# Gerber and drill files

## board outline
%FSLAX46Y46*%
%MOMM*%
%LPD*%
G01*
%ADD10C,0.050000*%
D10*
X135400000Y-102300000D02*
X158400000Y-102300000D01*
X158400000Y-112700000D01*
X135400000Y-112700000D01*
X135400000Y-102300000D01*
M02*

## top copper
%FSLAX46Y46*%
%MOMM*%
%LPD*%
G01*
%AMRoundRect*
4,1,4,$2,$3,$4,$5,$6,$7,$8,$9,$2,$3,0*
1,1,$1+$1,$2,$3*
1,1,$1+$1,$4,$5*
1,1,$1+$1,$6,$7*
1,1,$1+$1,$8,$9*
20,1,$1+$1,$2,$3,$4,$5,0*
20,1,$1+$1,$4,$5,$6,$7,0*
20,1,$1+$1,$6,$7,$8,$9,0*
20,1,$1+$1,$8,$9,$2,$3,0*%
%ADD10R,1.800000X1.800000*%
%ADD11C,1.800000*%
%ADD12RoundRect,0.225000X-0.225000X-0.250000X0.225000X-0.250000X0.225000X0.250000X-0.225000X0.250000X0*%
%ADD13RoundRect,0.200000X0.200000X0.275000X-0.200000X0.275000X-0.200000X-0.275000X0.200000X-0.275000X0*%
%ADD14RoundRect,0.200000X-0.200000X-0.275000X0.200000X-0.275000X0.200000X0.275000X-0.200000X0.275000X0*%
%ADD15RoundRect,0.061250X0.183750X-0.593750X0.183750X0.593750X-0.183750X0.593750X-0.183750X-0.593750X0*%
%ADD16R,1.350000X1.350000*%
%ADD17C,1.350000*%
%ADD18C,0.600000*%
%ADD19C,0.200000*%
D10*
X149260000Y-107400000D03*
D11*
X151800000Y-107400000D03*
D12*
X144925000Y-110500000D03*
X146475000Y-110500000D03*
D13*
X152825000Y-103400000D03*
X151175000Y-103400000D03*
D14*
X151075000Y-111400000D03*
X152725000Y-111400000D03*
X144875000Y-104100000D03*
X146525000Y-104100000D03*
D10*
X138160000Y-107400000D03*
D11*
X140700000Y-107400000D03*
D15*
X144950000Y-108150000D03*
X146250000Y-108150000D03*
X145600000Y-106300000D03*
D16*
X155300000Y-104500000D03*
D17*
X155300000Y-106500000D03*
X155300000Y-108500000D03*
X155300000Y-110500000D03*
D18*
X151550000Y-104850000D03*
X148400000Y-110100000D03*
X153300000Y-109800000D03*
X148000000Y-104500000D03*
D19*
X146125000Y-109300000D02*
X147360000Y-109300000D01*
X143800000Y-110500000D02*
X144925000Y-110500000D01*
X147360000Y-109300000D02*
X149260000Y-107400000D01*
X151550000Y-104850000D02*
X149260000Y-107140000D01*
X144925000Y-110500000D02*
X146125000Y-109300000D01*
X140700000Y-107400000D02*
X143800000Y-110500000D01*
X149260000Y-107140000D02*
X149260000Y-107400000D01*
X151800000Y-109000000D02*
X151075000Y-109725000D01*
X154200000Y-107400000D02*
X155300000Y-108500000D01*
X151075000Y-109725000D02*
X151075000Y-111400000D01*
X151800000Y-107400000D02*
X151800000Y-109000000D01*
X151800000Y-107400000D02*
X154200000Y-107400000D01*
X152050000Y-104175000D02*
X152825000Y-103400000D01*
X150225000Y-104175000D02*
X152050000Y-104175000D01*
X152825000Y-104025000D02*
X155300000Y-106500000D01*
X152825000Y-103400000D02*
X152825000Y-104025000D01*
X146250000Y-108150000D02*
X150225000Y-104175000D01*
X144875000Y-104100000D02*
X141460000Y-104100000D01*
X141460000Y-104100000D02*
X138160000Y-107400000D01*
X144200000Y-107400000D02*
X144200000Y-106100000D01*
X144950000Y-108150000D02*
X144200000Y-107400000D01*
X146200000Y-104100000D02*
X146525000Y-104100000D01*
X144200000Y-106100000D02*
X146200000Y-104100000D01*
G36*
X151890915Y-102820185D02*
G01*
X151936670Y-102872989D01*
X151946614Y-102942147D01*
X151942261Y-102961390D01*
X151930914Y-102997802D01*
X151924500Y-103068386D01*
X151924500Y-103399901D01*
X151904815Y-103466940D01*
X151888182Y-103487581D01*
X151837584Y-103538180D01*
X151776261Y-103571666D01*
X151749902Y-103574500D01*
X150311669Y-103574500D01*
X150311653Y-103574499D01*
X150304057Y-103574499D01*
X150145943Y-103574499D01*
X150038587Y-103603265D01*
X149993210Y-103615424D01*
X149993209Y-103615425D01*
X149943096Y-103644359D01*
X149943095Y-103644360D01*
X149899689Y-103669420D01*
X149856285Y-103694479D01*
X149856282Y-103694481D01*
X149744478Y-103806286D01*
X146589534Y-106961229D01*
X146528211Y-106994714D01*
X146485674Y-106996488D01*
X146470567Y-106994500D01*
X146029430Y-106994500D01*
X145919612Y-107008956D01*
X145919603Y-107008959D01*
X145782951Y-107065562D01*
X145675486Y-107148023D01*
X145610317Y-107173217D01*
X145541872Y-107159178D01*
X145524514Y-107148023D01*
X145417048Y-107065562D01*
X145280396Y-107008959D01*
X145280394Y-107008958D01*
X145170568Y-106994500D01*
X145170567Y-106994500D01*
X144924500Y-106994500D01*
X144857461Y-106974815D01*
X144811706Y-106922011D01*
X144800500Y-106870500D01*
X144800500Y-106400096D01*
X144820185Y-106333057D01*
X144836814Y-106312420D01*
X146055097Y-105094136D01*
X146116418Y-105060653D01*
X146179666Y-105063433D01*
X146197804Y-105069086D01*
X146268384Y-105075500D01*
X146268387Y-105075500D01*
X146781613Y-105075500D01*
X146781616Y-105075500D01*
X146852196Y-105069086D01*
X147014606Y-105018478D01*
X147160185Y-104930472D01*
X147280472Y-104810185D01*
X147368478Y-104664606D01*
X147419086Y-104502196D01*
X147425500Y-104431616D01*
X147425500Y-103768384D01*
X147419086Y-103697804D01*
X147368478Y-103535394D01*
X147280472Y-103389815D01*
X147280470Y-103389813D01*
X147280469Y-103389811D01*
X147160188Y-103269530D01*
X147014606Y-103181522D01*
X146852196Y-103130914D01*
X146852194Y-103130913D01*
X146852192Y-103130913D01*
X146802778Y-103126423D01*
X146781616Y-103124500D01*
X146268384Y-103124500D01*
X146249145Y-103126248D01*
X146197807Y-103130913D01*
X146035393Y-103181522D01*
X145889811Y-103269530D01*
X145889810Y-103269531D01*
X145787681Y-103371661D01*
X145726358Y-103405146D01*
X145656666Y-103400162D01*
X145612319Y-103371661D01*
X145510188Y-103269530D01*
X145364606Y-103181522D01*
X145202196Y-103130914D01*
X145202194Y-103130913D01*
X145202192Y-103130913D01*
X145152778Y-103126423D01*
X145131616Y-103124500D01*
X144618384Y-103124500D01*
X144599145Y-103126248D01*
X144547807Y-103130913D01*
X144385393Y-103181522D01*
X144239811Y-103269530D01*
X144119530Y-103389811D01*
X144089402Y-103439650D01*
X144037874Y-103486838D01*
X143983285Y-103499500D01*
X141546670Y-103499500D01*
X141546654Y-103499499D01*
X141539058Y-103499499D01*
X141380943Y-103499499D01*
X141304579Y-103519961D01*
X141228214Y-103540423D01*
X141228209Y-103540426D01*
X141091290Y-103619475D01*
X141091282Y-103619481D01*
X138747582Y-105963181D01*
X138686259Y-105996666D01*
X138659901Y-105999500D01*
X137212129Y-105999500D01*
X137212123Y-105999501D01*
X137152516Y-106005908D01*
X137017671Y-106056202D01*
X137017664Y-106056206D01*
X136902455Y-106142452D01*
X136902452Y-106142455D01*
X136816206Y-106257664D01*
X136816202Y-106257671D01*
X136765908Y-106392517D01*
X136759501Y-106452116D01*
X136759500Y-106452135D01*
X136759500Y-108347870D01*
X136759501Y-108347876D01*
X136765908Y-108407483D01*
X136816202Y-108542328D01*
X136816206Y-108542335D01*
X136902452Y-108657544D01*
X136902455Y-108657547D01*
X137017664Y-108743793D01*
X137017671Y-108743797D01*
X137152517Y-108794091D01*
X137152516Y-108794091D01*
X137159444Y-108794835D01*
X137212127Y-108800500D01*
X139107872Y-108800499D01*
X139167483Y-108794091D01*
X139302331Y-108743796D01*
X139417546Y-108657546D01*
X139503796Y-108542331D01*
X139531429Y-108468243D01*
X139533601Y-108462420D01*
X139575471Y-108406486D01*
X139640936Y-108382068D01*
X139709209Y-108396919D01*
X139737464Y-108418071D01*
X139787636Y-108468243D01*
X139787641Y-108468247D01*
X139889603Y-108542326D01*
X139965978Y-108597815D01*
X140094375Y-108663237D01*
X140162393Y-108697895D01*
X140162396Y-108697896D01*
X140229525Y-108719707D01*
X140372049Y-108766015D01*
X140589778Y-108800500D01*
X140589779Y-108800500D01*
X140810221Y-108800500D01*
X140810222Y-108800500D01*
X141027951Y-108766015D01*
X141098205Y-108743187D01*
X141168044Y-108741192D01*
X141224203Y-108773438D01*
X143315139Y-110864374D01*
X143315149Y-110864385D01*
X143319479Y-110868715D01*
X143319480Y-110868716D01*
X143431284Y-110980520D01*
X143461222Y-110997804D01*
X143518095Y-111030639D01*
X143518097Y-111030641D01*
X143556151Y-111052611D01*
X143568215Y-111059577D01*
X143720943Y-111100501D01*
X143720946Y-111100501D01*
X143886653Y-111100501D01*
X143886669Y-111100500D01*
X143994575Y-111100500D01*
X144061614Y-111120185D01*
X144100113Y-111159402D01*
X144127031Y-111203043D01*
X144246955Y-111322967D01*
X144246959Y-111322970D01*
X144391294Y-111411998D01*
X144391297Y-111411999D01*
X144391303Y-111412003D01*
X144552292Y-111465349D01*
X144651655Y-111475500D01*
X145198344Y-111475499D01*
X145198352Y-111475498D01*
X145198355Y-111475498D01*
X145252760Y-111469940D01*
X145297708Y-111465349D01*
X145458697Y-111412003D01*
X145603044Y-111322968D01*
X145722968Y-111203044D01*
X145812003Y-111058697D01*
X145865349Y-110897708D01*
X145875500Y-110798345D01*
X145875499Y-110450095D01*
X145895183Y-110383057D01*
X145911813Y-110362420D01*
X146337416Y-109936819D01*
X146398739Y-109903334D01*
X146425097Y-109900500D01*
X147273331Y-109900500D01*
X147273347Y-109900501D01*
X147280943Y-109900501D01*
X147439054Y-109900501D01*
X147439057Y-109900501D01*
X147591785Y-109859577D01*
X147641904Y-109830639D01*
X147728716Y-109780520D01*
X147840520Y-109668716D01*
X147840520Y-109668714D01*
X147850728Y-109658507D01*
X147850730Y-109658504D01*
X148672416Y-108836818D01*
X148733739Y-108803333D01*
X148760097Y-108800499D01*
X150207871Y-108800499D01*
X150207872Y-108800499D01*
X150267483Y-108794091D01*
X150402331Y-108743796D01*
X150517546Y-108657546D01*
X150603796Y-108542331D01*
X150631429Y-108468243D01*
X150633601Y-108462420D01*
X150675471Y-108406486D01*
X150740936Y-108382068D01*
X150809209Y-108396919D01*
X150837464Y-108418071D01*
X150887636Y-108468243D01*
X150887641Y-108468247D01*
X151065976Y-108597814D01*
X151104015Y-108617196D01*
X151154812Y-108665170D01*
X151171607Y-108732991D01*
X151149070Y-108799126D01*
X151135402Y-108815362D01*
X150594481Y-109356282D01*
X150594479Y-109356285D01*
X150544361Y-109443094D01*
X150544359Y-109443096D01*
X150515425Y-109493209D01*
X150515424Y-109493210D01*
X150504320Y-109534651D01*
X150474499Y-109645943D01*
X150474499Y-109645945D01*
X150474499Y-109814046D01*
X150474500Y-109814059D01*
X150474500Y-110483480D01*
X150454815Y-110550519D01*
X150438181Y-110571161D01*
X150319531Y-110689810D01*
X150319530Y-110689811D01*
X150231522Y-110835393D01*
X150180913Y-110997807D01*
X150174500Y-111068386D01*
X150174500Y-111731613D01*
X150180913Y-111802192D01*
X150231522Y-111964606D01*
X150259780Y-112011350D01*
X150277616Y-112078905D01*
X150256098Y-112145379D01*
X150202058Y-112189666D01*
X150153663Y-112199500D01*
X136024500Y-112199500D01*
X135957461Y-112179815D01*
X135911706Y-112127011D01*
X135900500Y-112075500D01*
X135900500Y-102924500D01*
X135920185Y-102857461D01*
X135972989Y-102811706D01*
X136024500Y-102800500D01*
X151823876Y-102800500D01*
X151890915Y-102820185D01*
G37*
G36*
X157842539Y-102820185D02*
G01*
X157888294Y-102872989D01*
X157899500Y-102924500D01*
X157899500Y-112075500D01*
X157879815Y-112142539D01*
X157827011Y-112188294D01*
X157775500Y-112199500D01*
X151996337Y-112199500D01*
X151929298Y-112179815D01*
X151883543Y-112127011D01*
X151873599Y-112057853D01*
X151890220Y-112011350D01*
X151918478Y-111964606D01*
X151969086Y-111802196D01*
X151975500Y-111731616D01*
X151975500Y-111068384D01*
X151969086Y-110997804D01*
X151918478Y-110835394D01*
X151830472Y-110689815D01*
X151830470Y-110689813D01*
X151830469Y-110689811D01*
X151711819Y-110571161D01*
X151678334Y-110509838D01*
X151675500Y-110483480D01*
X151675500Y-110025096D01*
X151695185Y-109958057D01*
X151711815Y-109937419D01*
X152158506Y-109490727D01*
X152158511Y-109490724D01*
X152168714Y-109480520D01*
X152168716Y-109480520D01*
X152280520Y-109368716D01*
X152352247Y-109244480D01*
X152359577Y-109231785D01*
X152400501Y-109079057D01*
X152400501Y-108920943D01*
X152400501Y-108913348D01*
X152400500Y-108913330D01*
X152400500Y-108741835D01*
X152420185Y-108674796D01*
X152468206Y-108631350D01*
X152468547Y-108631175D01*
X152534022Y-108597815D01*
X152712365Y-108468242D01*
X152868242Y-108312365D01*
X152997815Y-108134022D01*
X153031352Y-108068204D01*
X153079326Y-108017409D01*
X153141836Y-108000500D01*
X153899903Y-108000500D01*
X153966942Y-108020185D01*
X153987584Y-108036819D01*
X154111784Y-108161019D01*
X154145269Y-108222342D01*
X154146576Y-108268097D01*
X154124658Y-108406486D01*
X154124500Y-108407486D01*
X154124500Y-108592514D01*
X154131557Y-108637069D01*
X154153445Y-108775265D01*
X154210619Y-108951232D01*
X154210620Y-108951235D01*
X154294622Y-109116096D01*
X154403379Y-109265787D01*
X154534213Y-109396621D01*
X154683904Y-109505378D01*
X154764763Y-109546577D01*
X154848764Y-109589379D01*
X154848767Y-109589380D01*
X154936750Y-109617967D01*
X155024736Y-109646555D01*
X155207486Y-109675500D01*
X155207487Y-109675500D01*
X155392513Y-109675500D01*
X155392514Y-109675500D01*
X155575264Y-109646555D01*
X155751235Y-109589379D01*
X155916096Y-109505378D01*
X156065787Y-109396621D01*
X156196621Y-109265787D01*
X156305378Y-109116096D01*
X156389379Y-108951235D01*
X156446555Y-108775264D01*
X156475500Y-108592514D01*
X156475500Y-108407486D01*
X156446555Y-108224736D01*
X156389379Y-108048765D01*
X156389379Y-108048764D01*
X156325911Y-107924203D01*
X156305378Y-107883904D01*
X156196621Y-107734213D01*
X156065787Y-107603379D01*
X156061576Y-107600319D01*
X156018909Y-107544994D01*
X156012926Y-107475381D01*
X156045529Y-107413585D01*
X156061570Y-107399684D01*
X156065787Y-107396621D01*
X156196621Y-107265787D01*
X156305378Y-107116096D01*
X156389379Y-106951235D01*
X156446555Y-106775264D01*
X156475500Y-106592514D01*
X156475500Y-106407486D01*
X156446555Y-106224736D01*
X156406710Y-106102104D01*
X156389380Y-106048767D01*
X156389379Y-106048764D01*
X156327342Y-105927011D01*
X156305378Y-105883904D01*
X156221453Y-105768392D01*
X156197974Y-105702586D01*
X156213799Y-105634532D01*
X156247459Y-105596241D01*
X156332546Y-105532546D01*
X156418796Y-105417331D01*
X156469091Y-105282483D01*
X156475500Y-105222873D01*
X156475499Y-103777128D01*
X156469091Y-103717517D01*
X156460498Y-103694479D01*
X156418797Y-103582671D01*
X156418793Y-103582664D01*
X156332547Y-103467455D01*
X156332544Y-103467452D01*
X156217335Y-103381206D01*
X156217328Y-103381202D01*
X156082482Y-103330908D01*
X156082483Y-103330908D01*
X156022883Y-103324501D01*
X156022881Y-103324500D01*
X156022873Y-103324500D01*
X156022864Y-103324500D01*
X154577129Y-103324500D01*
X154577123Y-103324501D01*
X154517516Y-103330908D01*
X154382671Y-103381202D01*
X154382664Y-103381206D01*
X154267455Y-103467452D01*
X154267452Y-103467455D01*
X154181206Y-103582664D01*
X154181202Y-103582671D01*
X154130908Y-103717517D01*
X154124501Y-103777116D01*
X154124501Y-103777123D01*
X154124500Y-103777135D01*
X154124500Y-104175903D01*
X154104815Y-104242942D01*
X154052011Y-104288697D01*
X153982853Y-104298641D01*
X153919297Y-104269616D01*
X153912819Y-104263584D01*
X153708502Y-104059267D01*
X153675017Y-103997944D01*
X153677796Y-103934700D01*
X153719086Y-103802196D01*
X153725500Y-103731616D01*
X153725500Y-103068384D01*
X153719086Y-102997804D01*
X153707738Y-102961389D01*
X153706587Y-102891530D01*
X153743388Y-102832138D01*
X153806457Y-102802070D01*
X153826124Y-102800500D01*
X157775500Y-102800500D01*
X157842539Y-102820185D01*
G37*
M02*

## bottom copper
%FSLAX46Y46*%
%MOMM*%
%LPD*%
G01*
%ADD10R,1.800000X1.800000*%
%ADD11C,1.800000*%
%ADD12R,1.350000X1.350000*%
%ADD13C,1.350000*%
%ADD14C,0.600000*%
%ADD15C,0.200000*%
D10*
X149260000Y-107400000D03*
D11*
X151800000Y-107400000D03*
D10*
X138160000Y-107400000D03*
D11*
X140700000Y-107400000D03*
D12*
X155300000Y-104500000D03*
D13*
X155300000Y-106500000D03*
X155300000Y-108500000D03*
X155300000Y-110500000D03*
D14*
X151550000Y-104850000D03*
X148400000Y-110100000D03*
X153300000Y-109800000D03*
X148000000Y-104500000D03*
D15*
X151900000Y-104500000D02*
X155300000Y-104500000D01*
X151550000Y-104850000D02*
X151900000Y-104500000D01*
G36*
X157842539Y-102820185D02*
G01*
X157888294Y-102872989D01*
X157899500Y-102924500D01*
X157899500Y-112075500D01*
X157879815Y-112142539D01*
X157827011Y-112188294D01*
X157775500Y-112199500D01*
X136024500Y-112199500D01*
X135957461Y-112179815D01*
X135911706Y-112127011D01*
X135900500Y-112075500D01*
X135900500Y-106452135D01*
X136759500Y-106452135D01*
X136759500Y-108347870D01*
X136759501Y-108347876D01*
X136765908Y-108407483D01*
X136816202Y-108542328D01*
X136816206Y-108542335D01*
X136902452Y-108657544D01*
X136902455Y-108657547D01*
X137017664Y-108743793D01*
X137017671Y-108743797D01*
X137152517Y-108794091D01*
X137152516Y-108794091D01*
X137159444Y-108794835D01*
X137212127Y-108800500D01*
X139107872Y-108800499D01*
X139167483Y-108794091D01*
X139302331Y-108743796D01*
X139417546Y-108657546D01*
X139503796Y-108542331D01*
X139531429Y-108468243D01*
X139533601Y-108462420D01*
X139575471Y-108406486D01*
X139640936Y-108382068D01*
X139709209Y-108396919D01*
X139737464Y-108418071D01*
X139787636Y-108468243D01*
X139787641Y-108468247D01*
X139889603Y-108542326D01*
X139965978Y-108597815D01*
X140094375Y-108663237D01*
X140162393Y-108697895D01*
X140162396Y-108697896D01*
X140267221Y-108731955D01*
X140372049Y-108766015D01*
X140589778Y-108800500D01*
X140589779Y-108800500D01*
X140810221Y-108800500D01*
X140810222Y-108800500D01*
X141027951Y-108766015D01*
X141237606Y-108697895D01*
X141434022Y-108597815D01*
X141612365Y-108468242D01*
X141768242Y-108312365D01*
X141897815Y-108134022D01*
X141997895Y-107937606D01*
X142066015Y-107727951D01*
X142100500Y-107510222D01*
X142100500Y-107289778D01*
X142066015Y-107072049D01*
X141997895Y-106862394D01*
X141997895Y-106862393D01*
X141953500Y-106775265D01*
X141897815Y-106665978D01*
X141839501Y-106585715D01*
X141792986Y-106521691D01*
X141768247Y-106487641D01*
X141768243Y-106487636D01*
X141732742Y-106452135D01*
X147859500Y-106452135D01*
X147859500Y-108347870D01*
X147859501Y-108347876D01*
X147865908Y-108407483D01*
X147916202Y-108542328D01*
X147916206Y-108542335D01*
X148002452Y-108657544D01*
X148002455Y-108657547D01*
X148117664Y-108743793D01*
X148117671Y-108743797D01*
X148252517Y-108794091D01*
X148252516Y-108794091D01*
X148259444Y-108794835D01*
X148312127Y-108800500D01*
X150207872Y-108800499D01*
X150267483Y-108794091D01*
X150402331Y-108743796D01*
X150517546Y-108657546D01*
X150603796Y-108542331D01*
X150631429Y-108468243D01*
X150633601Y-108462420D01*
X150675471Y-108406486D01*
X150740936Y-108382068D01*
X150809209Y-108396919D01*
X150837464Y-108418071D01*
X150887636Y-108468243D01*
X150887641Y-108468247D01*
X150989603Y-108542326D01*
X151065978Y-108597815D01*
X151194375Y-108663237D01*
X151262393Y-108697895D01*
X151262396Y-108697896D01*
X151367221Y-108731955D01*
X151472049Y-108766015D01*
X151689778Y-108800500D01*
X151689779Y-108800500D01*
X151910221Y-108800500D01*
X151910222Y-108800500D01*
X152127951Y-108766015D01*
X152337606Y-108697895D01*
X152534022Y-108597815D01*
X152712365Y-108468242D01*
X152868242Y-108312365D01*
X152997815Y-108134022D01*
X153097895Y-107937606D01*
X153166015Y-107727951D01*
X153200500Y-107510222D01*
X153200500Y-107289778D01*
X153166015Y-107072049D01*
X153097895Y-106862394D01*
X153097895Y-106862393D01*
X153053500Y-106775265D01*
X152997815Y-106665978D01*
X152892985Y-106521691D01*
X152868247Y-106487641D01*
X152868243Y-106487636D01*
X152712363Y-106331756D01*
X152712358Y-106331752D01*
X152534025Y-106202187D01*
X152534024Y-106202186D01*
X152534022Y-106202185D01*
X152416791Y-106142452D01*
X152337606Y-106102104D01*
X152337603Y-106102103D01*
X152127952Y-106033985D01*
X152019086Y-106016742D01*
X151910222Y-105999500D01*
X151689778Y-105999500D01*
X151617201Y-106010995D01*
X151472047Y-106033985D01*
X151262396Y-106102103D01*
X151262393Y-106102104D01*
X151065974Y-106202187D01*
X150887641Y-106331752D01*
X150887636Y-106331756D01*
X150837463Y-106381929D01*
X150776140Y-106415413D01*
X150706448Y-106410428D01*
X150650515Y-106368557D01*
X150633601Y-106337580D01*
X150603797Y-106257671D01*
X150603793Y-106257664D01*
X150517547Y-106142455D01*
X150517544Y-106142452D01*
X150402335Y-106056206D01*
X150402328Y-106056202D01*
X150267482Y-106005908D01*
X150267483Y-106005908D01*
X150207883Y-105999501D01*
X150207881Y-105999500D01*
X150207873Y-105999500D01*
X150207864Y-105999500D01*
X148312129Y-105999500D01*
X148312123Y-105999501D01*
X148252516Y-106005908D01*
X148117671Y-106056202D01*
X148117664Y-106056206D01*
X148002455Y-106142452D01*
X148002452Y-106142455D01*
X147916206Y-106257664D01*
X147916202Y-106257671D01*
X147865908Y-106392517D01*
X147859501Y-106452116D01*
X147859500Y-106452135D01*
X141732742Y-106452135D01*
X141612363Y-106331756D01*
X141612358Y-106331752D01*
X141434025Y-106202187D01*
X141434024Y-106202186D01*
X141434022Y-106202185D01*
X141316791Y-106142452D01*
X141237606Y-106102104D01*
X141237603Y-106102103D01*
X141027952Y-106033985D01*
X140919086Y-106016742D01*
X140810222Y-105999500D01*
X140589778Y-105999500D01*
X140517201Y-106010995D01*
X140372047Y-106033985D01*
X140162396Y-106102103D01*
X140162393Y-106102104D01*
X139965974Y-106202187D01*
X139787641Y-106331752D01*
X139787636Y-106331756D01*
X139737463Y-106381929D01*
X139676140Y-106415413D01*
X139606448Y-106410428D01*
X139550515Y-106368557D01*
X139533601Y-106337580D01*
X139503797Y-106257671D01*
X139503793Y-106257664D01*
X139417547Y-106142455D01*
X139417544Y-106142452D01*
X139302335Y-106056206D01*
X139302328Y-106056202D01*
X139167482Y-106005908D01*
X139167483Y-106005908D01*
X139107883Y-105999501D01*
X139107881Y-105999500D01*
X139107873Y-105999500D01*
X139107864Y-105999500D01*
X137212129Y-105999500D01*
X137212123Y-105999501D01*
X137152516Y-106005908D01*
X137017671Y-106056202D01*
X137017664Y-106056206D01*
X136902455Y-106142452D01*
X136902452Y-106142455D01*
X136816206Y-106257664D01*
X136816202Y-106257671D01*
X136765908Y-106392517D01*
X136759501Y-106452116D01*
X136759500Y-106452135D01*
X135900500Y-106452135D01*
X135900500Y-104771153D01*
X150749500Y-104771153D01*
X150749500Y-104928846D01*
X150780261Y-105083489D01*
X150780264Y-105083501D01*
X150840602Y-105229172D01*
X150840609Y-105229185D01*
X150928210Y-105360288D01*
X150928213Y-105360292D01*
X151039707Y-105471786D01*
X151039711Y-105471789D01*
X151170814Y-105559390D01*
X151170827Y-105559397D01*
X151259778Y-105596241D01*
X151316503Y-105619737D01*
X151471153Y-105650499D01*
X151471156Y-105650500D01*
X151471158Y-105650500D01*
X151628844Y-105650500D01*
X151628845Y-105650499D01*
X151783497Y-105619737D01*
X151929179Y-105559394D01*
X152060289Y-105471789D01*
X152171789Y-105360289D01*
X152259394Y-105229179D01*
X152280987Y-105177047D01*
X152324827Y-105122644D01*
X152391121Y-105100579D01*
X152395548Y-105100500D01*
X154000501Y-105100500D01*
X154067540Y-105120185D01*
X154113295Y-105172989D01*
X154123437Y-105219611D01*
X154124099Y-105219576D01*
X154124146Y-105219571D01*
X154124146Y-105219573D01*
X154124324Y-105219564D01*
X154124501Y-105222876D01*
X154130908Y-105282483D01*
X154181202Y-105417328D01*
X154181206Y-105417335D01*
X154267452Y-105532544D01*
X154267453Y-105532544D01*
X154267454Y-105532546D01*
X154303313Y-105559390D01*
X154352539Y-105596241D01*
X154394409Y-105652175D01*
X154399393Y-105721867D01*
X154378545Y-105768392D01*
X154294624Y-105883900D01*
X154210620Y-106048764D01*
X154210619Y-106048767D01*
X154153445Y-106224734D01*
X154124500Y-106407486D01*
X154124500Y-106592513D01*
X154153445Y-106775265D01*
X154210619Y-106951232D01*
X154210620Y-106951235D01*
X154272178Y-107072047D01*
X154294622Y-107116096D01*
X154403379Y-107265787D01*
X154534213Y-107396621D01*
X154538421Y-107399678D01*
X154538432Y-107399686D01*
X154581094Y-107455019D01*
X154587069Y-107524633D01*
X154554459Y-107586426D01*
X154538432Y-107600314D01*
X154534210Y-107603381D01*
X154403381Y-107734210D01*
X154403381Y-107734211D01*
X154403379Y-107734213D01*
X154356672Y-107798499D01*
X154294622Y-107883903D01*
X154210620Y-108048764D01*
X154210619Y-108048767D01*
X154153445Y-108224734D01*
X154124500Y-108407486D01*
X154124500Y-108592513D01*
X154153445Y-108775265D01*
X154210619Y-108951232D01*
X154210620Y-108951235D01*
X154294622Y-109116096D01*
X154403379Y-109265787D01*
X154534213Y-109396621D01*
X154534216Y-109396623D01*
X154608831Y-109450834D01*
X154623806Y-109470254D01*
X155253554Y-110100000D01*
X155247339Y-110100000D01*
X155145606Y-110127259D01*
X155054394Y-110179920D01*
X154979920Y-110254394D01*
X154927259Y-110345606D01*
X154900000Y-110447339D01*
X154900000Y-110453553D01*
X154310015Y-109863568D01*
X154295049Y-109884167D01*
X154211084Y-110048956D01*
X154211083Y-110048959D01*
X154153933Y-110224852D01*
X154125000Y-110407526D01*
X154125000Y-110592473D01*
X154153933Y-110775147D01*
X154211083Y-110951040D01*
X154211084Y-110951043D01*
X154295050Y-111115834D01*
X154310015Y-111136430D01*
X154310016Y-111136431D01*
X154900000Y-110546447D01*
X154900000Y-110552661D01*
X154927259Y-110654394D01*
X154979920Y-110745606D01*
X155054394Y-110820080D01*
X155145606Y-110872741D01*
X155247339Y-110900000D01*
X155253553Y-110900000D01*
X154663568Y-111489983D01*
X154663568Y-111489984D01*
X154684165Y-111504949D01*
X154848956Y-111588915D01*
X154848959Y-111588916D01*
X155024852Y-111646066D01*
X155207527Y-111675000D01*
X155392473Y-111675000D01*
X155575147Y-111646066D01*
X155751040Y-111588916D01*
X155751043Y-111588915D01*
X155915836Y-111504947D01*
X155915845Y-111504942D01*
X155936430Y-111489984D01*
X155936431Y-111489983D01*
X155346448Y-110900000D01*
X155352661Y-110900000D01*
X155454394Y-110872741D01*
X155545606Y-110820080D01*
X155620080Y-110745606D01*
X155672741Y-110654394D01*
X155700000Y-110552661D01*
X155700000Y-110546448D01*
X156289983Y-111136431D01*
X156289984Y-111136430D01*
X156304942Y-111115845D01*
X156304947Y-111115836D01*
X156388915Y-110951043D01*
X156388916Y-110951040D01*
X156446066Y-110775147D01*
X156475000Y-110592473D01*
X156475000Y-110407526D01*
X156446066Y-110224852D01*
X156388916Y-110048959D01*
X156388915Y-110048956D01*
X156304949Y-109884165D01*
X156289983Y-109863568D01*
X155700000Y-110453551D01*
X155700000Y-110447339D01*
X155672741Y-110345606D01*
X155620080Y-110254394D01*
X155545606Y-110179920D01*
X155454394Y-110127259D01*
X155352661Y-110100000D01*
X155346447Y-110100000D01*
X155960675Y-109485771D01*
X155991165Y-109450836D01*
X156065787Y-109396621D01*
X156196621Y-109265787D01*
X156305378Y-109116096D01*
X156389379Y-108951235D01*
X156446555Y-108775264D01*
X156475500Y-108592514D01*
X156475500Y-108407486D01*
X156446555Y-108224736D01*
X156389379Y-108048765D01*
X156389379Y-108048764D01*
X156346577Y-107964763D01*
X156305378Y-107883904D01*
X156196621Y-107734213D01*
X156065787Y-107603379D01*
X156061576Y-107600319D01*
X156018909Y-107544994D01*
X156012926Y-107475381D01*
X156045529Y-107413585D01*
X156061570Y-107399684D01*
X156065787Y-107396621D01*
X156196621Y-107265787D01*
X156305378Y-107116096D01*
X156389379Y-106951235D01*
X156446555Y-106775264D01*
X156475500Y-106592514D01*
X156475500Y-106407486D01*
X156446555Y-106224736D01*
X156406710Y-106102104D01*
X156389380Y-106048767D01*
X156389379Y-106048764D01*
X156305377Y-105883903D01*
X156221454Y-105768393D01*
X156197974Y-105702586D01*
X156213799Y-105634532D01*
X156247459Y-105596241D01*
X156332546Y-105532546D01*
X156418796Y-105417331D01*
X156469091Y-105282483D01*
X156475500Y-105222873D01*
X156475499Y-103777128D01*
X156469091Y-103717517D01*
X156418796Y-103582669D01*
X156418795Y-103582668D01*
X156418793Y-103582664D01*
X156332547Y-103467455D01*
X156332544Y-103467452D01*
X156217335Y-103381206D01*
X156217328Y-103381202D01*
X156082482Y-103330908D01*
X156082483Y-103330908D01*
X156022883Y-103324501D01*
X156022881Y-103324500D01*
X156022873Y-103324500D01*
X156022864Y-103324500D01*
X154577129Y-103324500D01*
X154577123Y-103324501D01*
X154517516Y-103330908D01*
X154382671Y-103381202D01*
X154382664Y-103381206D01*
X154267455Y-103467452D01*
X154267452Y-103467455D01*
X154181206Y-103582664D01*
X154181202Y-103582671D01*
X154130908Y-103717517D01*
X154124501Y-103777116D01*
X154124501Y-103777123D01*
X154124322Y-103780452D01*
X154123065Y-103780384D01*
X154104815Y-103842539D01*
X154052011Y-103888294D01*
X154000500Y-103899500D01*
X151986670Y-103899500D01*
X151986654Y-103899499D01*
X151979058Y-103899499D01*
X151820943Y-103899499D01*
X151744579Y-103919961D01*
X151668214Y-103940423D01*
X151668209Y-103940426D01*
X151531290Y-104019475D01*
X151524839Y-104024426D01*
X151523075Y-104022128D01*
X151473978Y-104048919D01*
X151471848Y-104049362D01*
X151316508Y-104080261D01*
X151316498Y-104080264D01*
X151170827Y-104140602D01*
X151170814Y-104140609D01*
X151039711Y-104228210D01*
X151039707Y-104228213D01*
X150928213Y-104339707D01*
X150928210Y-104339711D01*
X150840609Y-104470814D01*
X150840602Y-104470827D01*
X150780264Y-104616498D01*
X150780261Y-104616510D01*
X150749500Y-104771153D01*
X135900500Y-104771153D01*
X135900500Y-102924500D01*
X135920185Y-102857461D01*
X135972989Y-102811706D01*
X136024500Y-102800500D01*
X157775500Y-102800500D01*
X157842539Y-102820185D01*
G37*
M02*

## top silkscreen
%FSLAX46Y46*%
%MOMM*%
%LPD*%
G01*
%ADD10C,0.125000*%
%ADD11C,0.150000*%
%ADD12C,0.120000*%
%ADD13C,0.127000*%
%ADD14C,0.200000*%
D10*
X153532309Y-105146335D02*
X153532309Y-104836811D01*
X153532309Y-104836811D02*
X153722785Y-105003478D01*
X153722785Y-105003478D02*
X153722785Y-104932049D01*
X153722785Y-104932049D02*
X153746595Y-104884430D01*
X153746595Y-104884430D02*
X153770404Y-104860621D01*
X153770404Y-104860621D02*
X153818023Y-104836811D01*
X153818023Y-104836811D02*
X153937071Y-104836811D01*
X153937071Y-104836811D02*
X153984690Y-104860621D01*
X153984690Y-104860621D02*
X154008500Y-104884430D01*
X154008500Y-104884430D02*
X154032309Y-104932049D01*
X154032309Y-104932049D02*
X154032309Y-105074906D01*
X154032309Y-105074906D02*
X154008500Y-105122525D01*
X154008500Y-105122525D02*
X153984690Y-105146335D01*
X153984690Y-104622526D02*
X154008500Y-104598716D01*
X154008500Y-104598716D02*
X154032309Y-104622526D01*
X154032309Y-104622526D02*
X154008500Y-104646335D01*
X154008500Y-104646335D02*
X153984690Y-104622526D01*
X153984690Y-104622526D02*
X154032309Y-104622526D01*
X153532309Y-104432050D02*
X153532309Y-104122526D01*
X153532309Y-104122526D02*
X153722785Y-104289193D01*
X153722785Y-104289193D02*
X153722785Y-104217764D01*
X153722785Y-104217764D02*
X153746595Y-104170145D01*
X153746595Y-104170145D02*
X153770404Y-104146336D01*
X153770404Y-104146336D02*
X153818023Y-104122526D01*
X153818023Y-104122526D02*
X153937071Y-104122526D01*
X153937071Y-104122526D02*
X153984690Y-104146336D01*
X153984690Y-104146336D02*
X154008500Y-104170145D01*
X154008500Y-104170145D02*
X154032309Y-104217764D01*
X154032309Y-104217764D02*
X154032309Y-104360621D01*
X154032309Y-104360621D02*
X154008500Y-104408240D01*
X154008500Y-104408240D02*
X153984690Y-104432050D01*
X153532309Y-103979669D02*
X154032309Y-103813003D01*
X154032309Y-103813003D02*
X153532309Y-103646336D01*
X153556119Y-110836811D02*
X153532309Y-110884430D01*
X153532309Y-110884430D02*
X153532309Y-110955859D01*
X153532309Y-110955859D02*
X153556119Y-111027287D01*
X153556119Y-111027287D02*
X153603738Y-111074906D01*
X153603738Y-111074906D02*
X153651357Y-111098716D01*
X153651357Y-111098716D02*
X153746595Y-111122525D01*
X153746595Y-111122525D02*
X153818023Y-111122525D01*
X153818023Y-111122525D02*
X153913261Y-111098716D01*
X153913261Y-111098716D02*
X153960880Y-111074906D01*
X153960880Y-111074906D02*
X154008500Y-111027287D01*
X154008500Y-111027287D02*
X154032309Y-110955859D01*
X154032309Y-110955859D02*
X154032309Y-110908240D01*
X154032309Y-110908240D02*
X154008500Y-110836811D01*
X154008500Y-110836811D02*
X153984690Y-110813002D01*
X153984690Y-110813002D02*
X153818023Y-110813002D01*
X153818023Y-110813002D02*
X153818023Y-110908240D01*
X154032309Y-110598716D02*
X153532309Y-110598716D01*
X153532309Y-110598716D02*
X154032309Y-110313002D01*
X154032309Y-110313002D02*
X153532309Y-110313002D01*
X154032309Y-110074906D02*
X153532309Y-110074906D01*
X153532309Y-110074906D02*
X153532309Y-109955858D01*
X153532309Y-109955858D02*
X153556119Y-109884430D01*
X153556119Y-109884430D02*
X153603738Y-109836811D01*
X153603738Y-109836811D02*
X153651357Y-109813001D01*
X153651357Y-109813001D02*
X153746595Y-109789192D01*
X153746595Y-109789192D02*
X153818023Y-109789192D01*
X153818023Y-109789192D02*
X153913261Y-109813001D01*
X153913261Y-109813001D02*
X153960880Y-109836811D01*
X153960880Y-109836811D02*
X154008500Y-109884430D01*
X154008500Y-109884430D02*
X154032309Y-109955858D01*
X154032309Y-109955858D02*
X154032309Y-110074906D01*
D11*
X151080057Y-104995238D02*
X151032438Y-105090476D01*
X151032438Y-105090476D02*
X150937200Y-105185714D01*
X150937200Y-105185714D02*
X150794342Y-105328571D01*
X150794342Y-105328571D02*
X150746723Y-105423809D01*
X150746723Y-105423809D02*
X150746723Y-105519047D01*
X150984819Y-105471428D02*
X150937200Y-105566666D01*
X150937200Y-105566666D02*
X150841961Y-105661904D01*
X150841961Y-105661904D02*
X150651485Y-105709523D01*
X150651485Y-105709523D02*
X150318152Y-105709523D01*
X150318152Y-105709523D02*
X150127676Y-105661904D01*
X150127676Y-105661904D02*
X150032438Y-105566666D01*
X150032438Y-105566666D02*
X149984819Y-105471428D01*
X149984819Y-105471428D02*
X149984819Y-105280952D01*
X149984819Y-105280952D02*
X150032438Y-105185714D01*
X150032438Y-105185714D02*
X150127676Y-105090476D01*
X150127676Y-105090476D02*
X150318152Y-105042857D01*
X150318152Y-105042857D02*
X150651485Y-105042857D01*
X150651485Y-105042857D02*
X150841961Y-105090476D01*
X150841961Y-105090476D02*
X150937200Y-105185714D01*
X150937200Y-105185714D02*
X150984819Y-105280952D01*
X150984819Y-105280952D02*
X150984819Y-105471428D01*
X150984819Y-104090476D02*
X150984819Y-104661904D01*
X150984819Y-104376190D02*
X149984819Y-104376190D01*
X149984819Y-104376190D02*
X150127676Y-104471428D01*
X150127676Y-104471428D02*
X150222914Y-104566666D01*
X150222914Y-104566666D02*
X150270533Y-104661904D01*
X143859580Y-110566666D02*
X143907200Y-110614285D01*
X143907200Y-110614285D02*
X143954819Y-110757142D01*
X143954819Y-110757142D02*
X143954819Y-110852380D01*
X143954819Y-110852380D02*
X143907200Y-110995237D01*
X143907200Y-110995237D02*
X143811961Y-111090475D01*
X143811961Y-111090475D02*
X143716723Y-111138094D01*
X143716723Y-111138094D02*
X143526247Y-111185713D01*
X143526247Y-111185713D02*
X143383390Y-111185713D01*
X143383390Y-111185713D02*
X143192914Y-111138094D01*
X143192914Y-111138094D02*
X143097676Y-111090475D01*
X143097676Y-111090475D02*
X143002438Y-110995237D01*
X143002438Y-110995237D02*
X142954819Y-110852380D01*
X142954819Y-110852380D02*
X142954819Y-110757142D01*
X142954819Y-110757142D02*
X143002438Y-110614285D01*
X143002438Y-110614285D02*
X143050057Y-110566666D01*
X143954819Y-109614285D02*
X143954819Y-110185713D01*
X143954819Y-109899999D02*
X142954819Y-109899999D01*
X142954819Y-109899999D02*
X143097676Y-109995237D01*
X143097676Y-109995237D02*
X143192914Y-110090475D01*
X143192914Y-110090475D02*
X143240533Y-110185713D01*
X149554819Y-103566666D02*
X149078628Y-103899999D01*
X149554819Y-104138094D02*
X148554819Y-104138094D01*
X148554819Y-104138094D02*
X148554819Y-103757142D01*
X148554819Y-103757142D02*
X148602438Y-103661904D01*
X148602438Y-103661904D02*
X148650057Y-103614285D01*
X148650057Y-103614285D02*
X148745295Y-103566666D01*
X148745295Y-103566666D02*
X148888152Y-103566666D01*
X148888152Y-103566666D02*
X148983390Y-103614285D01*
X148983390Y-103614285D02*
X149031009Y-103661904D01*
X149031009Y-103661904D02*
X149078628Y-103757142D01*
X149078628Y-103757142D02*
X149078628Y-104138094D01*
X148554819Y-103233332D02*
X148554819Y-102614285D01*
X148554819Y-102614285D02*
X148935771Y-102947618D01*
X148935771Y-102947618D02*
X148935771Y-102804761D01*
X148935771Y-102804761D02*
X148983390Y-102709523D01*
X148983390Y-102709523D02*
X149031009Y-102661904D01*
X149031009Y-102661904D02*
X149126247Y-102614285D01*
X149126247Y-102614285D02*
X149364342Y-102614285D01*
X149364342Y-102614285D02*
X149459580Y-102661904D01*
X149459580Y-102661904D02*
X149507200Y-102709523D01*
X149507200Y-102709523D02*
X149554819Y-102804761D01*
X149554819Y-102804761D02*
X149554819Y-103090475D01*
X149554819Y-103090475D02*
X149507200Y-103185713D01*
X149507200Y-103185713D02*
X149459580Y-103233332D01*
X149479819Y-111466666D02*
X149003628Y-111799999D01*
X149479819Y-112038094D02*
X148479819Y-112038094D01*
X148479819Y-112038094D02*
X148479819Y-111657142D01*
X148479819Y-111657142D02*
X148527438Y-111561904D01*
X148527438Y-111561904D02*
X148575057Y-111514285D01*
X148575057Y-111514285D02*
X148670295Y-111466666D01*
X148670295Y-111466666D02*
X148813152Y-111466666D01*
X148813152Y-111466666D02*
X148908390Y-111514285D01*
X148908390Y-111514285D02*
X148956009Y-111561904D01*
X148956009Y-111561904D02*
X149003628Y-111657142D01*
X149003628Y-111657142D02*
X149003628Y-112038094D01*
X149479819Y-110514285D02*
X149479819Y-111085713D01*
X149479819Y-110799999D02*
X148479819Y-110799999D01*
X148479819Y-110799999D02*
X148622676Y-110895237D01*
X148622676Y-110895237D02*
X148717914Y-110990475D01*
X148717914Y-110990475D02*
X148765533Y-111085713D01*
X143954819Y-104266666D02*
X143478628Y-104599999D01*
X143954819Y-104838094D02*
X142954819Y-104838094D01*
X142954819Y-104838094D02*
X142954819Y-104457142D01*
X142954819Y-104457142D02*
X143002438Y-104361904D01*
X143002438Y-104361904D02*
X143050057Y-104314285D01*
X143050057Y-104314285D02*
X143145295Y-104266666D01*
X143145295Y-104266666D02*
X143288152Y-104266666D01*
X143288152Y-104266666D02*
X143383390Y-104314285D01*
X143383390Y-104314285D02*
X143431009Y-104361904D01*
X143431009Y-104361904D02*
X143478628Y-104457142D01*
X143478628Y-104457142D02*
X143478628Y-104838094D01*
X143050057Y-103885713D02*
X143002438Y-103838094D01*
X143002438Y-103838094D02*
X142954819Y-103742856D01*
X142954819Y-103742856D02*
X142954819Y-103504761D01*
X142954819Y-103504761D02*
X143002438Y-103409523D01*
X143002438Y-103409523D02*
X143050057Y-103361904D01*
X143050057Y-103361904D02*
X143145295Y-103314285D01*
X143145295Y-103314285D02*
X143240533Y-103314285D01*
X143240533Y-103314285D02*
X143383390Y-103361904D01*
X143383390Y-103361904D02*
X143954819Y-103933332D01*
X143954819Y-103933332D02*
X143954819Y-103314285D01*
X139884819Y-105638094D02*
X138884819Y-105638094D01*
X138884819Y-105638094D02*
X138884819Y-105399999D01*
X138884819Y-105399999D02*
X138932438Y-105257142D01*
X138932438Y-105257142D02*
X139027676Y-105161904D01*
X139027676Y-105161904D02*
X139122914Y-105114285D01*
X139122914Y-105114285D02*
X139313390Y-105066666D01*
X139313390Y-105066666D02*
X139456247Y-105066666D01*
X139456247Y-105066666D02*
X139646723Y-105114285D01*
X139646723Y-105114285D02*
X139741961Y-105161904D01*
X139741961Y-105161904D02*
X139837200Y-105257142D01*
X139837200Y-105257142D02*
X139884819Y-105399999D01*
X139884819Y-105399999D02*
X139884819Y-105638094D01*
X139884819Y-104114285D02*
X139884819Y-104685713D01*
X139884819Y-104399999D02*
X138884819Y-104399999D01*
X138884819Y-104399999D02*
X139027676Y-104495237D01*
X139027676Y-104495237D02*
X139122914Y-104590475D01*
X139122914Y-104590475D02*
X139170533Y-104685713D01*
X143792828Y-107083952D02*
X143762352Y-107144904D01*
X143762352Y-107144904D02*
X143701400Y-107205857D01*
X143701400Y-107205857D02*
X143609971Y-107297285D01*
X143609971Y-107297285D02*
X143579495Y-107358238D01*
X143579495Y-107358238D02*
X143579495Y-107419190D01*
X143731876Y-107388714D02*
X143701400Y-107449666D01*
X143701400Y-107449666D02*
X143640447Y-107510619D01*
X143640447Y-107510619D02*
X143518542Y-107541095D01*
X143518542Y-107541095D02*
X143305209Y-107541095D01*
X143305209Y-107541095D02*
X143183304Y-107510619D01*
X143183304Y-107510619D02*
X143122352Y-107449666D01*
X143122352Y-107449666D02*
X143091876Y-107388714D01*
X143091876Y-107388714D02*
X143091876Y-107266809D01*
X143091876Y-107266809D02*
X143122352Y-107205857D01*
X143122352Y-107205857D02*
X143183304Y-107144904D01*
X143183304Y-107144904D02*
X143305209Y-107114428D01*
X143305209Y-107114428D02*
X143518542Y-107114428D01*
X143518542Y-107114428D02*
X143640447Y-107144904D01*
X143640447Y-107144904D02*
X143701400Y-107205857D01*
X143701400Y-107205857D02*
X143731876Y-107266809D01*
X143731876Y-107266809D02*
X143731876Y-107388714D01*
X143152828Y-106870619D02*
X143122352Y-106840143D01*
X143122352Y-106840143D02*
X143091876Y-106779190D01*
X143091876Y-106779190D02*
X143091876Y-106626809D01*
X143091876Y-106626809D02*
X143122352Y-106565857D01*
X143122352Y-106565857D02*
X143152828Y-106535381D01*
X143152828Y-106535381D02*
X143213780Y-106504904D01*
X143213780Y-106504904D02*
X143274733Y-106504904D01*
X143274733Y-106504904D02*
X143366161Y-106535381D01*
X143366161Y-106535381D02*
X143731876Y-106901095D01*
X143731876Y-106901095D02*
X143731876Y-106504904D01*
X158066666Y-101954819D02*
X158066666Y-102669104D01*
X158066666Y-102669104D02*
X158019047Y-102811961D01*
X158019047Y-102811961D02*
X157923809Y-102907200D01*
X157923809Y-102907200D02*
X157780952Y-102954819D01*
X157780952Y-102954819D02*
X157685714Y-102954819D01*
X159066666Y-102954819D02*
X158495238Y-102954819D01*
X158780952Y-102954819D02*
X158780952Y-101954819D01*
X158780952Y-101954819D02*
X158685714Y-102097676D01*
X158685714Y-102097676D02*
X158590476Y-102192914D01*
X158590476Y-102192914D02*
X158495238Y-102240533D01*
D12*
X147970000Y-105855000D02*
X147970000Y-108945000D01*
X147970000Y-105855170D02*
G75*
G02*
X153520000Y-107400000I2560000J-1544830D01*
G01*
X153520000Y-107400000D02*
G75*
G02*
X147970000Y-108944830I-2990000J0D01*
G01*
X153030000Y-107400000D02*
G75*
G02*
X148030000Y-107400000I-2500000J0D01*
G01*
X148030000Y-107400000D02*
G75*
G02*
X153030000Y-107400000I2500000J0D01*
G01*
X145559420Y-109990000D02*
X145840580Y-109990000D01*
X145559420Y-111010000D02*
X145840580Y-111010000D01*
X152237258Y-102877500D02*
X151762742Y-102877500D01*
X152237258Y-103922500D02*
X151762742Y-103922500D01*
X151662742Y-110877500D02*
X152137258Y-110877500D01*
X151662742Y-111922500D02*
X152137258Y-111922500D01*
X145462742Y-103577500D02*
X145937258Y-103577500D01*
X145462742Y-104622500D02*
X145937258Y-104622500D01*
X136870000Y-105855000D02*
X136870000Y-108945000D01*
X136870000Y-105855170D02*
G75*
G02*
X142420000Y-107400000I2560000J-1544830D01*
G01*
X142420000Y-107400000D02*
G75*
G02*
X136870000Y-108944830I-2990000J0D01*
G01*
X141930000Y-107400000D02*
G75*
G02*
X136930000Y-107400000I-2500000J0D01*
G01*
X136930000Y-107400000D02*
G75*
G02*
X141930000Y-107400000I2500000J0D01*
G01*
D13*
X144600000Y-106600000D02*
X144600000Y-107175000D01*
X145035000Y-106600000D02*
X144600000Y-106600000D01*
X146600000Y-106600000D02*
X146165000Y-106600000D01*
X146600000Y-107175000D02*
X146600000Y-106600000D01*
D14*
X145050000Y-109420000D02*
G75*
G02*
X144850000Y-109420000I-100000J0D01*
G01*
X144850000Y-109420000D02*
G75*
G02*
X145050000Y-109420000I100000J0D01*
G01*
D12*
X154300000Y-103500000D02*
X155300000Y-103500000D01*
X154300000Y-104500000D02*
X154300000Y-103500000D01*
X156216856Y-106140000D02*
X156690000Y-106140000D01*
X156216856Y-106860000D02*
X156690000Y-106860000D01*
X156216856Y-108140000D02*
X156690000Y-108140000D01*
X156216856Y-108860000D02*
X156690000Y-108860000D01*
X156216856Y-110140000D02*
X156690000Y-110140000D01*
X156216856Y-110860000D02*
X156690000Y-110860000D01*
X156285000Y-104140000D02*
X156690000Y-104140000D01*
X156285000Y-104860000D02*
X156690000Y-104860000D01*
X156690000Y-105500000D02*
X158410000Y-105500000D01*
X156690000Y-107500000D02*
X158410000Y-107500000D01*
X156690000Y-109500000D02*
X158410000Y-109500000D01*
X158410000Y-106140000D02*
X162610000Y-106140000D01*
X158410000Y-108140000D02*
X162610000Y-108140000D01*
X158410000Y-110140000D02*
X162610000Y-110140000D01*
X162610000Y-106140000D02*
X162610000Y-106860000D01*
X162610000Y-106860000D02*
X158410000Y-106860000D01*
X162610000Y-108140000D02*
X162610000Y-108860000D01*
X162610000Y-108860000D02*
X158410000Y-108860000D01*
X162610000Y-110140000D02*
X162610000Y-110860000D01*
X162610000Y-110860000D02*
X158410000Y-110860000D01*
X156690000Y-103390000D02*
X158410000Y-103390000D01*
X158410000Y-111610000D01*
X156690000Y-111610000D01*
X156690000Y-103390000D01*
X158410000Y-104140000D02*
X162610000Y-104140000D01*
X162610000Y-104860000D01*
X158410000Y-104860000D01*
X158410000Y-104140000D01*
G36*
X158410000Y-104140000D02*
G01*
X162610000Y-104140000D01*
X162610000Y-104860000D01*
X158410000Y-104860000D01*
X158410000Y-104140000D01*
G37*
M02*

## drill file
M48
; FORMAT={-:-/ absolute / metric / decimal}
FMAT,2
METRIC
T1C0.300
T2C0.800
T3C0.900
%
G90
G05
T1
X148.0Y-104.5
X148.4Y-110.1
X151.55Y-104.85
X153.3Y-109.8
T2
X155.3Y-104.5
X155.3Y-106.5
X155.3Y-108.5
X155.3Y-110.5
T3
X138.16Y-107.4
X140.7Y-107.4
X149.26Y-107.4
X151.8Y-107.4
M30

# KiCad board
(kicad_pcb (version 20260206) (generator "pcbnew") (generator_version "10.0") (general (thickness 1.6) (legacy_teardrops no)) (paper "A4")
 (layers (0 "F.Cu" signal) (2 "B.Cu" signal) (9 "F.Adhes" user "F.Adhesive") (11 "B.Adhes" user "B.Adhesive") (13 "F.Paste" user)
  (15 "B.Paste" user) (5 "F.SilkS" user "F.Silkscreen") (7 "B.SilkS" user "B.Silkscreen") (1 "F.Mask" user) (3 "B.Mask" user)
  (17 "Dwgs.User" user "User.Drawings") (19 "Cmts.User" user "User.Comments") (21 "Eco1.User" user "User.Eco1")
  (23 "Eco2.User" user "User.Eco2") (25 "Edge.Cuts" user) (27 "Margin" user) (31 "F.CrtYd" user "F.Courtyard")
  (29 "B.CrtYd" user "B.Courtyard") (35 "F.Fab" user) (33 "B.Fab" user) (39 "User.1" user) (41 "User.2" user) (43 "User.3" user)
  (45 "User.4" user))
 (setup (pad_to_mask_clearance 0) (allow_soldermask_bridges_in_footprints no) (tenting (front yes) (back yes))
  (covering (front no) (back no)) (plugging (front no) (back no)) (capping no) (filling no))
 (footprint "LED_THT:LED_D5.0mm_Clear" (layer "F.Cu") (at 149.26 107.4)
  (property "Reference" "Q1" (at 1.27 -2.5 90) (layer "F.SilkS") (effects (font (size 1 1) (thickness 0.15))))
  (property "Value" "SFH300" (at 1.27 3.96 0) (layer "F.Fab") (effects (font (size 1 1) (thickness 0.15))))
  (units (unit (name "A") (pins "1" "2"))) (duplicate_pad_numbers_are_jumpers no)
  (fp_line (start -1.29 -1.545) (end -1.29 1.545) (stroke (width 0.12) (type solid)) (layer "F.SilkS"))
  (fp_arc (start -1.29 -1.54483) (mid 2.071779 -2.880495) (end 4.26 0) (stroke (width 0.12) (type solid)) (layer "F.SilkS"))
  (fp_arc (start 4.26 0) (mid 2.071779 2.880495) (end -1.29 1.54483) (stroke (width 0.12) (type solid)) (layer "F.SilkS"))
  (fp_circle (center 1.27 0) (end 3.77 0) (stroke (width 0.12) (type solid)) (fill no) (layer "F.SilkS"))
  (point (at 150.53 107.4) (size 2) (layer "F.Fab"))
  (pad "1" thru_hole rect (at 0 0) (size 1.8 1.8) (drill 0.9) (layers "*.Cu" "*.Mask") (remove_unused_layers no) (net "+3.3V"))
  (pad "2" thru_hole circle (at 2.54 0) (size 1.8 1.8) (drill 0.9) (layers "*.Cu" "*.Mask") (remove_unused_layers no) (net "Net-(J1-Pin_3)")))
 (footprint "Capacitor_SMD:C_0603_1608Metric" (layer "F.Cu") (at 145.7 110.5)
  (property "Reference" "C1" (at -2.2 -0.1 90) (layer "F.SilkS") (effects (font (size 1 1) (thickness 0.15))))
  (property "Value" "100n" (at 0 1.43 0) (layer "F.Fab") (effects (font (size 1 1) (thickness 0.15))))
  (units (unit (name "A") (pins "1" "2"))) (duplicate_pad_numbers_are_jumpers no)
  (fp_line (start -0.14058 -0.51) (end 0.14058 -0.51) (stroke (width 0.12) (type solid)) (layer "F.SilkS"))
  (fp_line (start -0.14058 0.51) (end 0.14058 0.51) (stroke (width 0.12) (type solid)) (layer "F.SilkS"))
  (pad "1" smd roundrect (at -0.775 0) (size 0.9 0.95) (layers "F.Cu" "F.Mask" "F.Paste") (roundrect_rratio 0.25) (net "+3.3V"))
  (pad "2" smd roundrect (at 0.775 0) (size 0.9 0.95) (layers "F.Cu" "F.Mask" "F.Paste") (roundrect_rratio 0.25) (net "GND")))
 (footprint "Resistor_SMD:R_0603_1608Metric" (layer "F.Cu") (at 152 103.4 180)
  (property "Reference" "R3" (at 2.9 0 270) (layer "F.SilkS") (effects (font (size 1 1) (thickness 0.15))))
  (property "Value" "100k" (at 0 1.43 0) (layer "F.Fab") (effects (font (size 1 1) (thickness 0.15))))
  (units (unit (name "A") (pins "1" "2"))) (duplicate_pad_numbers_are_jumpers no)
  (fp_line (start -0.237258 0.5225) (end 0.237258 0.5225) (stroke (width 0.12) (type solid)) (layer "F.SilkS"))
  (fp_line (start -0.237258 -0.5225) (end 0.237258 -0.5225) (stroke (width 0.12) (type solid)) (layer "F.SilkS"))
  (pad "1" smd roundrect (at -0.825 0 180) (size 0.8 0.95) (layers "F.Cu" "F.Mask" "F.Paste") (roundrect_rratio 0.25) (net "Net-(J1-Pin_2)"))
  (pad "2" smd roundrect (at 0.825 0 180) (size 0.8 0.95) (layers "F.Cu" "F.Mask" "F.Paste") (roundrect_rratio 0.25) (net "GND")))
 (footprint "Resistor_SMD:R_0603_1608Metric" (layer "F.Cu") (at 151.9 111.4)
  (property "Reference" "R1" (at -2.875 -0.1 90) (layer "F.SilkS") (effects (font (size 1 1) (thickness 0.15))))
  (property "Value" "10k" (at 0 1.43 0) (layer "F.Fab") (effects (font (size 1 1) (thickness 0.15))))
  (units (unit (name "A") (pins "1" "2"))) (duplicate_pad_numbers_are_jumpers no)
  (fp_line (start -0.237258 -0.5225) (end 0.237258 -0.5225) (stroke (width 0.12) (type solid)) (layer "F.SilkS"))
  (fp_line (start -0.237258 0.5225) (end 0.237258 0.5225) (stroke (width 0.12) (type solid)) (layer "F.SilkS"))
  (pad "1" smd roundrect (at -0.825 0) (size 0.8 0.95) (layers "F.Cu" "F.Mask" "F.Paste") (roundrect_rratio 0.25) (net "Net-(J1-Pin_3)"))
  (pad "2" smd roundrect (at 0.825 0) (size 0.8 0.95) (layers "F.Cu" "F.Mask" "F.Paste") (roundrect_rratio 0.25) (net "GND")))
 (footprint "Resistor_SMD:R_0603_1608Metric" (layer "F.Cu") (at 145.7 104.1)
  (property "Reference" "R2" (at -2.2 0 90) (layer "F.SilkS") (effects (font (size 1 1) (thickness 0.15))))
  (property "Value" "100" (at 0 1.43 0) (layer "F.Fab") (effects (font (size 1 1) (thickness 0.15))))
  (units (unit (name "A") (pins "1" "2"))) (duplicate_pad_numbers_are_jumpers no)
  (fp_line (start -0.237258 -0.5225) (end 0.237258 -0.5225) (stroke (width 0.12) (type solid)) (layer "F.SilkS"))
  (fp_line (start -0.237258 0.5225) (end 0.237258 0.5225) (stroke (width 0.12) (type solid)) (layer "F.SilkS"))
  (pad "1" smd roundrect (at -0.825 0) (size 0.8 0.95) (layers "F.Cu" "F.Mask" "F.Paste") (roundrect_rratio 0.25) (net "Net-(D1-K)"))
  (pad "2" smd roundrect (at 0.825 0) (size 0.8 0.95) (layers "F.Cu" "F.Mask" "F.Paste") (roundrect_rratio 0.25) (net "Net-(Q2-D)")))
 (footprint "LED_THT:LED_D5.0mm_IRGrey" (layer "F.Cu") (at 138.16 107.4)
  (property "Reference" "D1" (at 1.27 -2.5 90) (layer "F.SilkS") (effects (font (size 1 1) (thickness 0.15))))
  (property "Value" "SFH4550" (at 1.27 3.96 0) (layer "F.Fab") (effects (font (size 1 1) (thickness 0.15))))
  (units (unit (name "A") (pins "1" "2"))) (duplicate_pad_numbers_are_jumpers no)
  (fp_line (start -1.29 -1.545) (end -1.29 1.545) (stroke (width 0.12) (type solid)) (layer "F.SilkS"))
  (fp_arc (start -1.29 -1.54483) (mid 2.071779 -2.880495) (end 4.26 0) (stroke (width 0.12) (type solid)) (layer "F.SilkS"))
  (fp_arc (start 4.26 0) (mid 2.071779 2.880495) (end -1.29 1.54483) (stroke (width 0.12) (type solid)) (layer "F.SilkS"))
  (fp_circle (center 1.27 0) (end 3.77 0) (stroke (width 0.12) (type solid)) (fill no) (layer "F.SilkS"))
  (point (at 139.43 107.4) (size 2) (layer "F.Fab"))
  (pad "1" thru_hole rect (at 0 0) (size 1.8 1.8) (drill 0.9) (layers "*.Cu" "*.Mask") (remove_unused_layers no) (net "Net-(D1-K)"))
  (pad "2" thru_hole circle (at 2.54 0) (size 1.8 1.8) (drill 0.9) (layers "*.Cu" "*.Mask") (remove_unused_layers no) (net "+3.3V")))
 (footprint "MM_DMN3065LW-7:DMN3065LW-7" (layer "F.Cu") (at 145.6 107.225 90)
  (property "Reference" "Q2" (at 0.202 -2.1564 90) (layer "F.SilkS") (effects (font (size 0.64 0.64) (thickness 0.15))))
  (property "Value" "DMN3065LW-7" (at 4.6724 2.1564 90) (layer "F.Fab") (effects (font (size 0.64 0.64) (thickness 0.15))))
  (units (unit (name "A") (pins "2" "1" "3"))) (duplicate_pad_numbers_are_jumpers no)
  (fp_line (start 0.625 -1) (end 0.05 -1) (stroke (width 0.127) (type solid)) (layer "F.SilkS"))
  (fp_line (start 0.625 -0.565) (end 0.625 -1) (stroke (width 0.127) (type solid)) (layer "F.SilkS"))
  (fp_line (start 0.625 1) (end 0.625 0.565) (stroke (width 0.127) (type solid)) (layer "F.SilkS"))
  (fp_line (start 0.05 1) (end 0.625 1) (stroke (width 0.127) (type solid)) (layer "F.SilkS"))
  (fp_circle (center -2.195 -0.65) (end -2.095 -0.65) (stroke (width 0.2) (type solid)) (fill no) (layer "F.SilkS"))
  (pad "1" smd roundrect (at -0.925 -0.65 90) (size 1.31 0.49) (layers "F.Cu" "F.Mask" "F.Paste") (roundrect_rratio 0.125)
   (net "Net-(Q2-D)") (solder_mask_margin 0.102))
  (pad "2" smd roundrect (at -0.925 0.65 90) (size 1.31 0.49) (layers "F.Cu" "F.Mask" "F.Paste") (roundrect_rratio 0.125)
   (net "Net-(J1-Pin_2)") (solder_mask_margin 0.102))
  (pad "3" smd roundrect (at 0.925 0 90) (size 1.31 0.49) (layers "F.Cu" "F.Mask" "F.Paste") (roundrect_rratio 0.125) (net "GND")
   (solder_mask_margin 0.102)))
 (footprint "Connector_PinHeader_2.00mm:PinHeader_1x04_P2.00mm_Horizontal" (layer "F.Cu") (at 155.3 104.5)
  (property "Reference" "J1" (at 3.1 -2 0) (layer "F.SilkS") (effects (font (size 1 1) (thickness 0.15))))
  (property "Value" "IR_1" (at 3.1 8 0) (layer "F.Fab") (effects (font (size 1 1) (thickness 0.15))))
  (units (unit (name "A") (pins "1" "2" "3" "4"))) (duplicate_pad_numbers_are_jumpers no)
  (fp_line (start -1 -1) (end 0 -1) (stroke (width 0.12) (type solid)) (layer "F.SilkS"))
  (fp_line (start -1 0) (end -1 -1) (stroke (width 0.12) (type solid)) (layer "F.SilkS"))
  (fp_line (start 0.916856 1.64) (end 1.39 1.64) (stroke (width 0.12) (type solid)) (layer "F.SilkS"))
  (fp_line (start 0.916856 2.36) (end 1.39 2.36) (stroke (width 0.12) (type solid)) (layer "F.SilkS"))
  (fp_line (start 0.916856 3.64) (end 1.39 3.64) (stroke (width 0.12) (type solid)) (layer "F.SilkS"))
  (fp_line (start 0.916856 4.36) (end 1.39 4.36) (stroke (width 0.12) (type solid)) (layer "F.SilkS"))
  (fp_line (start 0.916856 5.64) (end 1.39 5.64) (stroke (width 0.12) (type solid)) (layer "F.SilkS"))
  (fp_line (start 0.916856 6.36) (end 1.39 6.36) (stroke (width 0.12) (type solid)) (layer "F.SilkS"))
  (fp_line (start 0.985 -0.36) (end 1.39 -0.36) (stroke (width 0.12) (type solid)) (layer "F.SilkS"))
  (fp_line (start 0.985 0.36) (end 1.39 0.36) (stroke (width 0.12) (type solid)) (layer "F.SilkS"))
  (fp_line (start 1.39 1) (end 3.11 1) (stroke (width 0.12) (type solid)) (layer "F.SilkS"))
  (fp_line (start 1.39 3) (end 3.11 3) (stroke (width 0.12) (type solid)) (layer "F.SilkS"))
  (fp_line (start 1.39 5) (end 3.11 5) (stroke (width 0.12) (type solid)) (layer "F.SilkS"))
  (fp_line (start 3.11 1.64) (end 7.31 1.64) (stroke (width 0.12) (type solid)) (layer "F.SilkS"))
  (fp_line (start 3.11 3.64) (end 7.31 3.64) (stroke (width 0.12) (type solid)) (layer "F.SilkS"))
  (fp_line (start 3.11 5.64) (end 7.31 5.64) (stroke (width 0.12) (type solid)) (layer "F.SilkS"))
  (fp_line (start 7.31 1.64) (end 7.31 2.36) (stroke (width 0.12) (type solid)) (layer "F.SilkS"))
  (fp_line (start 7.31 2.36) (end 3.11 2.36) (stroke (width 0.12) (type solid)) (layer "F.SilkS"))
  (fp_line (start 7.31 3.64) (end 7.31 4.36) (stroke (width 0.12) (type solid)) (layer "F.SilkS"))
  (fp_line (start 7.31 4.36) (end 3.11 4.36) (stroke (width 0.12) (type solid)) (layer "F.SilkS"))
  (fp_line (start 7.31 5.64) (end 7.31 6.36) (stroke (width 0.12) (type solid)) (layer "F.SilkS"))
  (fp_line (start 7.31 6.36) (end 3.11 6.36) (stroke (width 0.12) (type solid)) (layer "F.SilkS"))
  (fp_rect (start 1.39 -1.11) (end 3.11 7.11) (stroke (width 0.12) (type solid)) (fill no) (layer "F.SilkS"))
  (fp_rect (start 3.11 -0.36) (end 7.31 0.36) (stroke (width 0.12) (type solid)) (fill yes) (layer "F.SilkS"))
  (pad "1" thru_hole rect (at 0 0) (size 1.35 1.35) (drill 0.8) (layers "*.Cu" "*.Mask") (remove_unused_layers no) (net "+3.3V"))
  (pad "2" thru_hole circle (at 0 2) (size 1.35 1.35) (drill 0.8) (layers "*.Cu" "*.Mask") (remove_unused_layers no) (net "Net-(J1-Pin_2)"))
  (pad "3" thru_hole circle (at 0 4) (size 1.35 1.35) (drill 0.8) (layers "*.Cu" "*.Mask") (remove_unused_layers no) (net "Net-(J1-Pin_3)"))
  (pad "4" thru_hole circle (at 0 6) (size 1.35 1.35) (drill 0.8) (layers "*.Cu" "*.Mask") (remove_unused_layers no) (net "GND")))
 (gr_rect (start 135.4 102.3) (end 158.4 112.7) (stroke (width 0.05) (type solid)) (fill no) (layer "Edge.Cuts"))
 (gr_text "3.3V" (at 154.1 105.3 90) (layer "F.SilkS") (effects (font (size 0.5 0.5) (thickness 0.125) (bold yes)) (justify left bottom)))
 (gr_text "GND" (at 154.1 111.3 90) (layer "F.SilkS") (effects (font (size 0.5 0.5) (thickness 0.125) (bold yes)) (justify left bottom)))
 (segment (start 146.125 109.3) (end 147.36 109.3) (width 0.2) (layer "F.Cu") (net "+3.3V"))
 (segment (start 143.8 110.5) (end 144.925 110.5) (width 0.2) (layer "F.Cu") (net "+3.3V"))
 (segment (start 147.36 109.3) (end 149.26 107.4) (width 0.2) (layer "F.Cu") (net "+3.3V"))
 (segment (start 151.55 104.85) (end 149.26 107.14) (width 0.2) (layer "F.Cu") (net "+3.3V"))
 (segment (start 144.925 110.5) (end 146.125 109.3) (width 0.2) (layer "F.Cu") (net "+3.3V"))
 (segment (start 140.7 107.4) (end 143.8 110.5) (width 0.2) (layer "F.Cu") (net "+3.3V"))
 (segment (start 149.26 107.14) (end 149.26 107.4) (width 0.2) (layer "F.Cu") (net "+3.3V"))
 (via (at 151.55 104.85) (size 0.6) (drill 0.3) (layers "F.Cu" "B.Cu") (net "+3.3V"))
 (segment (start 151.9 104.5) (end 155.3 104.5) (width 0.2) (layer "B.Cu") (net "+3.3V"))
 (segment (start 151.55 104.85) (end 151.9 104.5) (width 0.2) (layer "B.Cu") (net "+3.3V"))
 (segment (start 151.8 109) (end 151.075 109.725) (width 0.2) (layer "F.Cu") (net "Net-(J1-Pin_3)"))
 (segment (start 154.2 107.4) (end 155.3 108.5) (width 0.2) (layer "F.Cu") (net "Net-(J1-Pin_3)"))
 (segment (start 151.075 109.725) (end 151.075 111.4) (width 0.2) (layer "F.Cu") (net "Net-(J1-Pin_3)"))
 (segment (start 151.8 107.4) (end 151.8 109) (width 0.2) (layer "F.Cu") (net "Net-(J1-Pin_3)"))
 (segment (start 151.8 107.4) (end 154.2 107.4) (width 0.2) (layer "F.Cu") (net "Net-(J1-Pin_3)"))
 (via (at 148.4 110.1) (size 0.6) (drill 0.3) (layers "F.Cu" "B.Cu") (free yes) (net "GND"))
 (via (at 153.3 109.8) (size 0.6) (drill 0.3) (layers "F.Cu" "B.Cu") (free yes) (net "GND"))
 (via (at 148 104.5) (size 0.6) (drill 0.3) (layers "F.Cu" "B.Cu") (free yes) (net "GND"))
 (segment (start 152.05 104.175) (end 152.825 103.4) (width 0.2) (layer "F.Cu") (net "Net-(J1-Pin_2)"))
 (segment (start 150.225 104.175) (end 152.05 104.175) (width 0.2) (layer "F.Cu") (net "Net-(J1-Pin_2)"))
 (segment (start 152.825 104.025) (end 155.3 106.5) (width 0.2) (layer "F.Cu") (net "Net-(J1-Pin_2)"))
 (segment (start 152.825 103.4) (end 152.825 104.025) (width 0.2) (layer "F.Cu") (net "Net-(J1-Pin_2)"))
 (segment (start 146.25 108.15) (end 150.225 104.175) (width 0.2) (layer "F.Cu") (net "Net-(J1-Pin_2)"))
 (segment (start 144.875 104.1) (end 141.46 104.1) (width 0.2) (layer "F.Cu") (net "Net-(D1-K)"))
 (segment (start 141.46 104.1) (end 138.16 107.4) (width 0.2) (layer "F.Cu") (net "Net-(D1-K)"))
 (segment (start 144.2 107.4) (end 144.2 106.1) (width 0.2) (layer "F.Cu") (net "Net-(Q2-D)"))
 (segment (start 144.95 108.15) (end 144.2 107.4) (width 0.2) (layer "F.Cu") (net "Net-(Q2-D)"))
 (segment (start 146.2 104.1) (end 146.525 104.1) (width 0.2) (layer "F.Cu") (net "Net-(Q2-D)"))
 (segment (start 144.2 106.1) (end 146.2 104.1) (width 0.2) (layer "F.Cu") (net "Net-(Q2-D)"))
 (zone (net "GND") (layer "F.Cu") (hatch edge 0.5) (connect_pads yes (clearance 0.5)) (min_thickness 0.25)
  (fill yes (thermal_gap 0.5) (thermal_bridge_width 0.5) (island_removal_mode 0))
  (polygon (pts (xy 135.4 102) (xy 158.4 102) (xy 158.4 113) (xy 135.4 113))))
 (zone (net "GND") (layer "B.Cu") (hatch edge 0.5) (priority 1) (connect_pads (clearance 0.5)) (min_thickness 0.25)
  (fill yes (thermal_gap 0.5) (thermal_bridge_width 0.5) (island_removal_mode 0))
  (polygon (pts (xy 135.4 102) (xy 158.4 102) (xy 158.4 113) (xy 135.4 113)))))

